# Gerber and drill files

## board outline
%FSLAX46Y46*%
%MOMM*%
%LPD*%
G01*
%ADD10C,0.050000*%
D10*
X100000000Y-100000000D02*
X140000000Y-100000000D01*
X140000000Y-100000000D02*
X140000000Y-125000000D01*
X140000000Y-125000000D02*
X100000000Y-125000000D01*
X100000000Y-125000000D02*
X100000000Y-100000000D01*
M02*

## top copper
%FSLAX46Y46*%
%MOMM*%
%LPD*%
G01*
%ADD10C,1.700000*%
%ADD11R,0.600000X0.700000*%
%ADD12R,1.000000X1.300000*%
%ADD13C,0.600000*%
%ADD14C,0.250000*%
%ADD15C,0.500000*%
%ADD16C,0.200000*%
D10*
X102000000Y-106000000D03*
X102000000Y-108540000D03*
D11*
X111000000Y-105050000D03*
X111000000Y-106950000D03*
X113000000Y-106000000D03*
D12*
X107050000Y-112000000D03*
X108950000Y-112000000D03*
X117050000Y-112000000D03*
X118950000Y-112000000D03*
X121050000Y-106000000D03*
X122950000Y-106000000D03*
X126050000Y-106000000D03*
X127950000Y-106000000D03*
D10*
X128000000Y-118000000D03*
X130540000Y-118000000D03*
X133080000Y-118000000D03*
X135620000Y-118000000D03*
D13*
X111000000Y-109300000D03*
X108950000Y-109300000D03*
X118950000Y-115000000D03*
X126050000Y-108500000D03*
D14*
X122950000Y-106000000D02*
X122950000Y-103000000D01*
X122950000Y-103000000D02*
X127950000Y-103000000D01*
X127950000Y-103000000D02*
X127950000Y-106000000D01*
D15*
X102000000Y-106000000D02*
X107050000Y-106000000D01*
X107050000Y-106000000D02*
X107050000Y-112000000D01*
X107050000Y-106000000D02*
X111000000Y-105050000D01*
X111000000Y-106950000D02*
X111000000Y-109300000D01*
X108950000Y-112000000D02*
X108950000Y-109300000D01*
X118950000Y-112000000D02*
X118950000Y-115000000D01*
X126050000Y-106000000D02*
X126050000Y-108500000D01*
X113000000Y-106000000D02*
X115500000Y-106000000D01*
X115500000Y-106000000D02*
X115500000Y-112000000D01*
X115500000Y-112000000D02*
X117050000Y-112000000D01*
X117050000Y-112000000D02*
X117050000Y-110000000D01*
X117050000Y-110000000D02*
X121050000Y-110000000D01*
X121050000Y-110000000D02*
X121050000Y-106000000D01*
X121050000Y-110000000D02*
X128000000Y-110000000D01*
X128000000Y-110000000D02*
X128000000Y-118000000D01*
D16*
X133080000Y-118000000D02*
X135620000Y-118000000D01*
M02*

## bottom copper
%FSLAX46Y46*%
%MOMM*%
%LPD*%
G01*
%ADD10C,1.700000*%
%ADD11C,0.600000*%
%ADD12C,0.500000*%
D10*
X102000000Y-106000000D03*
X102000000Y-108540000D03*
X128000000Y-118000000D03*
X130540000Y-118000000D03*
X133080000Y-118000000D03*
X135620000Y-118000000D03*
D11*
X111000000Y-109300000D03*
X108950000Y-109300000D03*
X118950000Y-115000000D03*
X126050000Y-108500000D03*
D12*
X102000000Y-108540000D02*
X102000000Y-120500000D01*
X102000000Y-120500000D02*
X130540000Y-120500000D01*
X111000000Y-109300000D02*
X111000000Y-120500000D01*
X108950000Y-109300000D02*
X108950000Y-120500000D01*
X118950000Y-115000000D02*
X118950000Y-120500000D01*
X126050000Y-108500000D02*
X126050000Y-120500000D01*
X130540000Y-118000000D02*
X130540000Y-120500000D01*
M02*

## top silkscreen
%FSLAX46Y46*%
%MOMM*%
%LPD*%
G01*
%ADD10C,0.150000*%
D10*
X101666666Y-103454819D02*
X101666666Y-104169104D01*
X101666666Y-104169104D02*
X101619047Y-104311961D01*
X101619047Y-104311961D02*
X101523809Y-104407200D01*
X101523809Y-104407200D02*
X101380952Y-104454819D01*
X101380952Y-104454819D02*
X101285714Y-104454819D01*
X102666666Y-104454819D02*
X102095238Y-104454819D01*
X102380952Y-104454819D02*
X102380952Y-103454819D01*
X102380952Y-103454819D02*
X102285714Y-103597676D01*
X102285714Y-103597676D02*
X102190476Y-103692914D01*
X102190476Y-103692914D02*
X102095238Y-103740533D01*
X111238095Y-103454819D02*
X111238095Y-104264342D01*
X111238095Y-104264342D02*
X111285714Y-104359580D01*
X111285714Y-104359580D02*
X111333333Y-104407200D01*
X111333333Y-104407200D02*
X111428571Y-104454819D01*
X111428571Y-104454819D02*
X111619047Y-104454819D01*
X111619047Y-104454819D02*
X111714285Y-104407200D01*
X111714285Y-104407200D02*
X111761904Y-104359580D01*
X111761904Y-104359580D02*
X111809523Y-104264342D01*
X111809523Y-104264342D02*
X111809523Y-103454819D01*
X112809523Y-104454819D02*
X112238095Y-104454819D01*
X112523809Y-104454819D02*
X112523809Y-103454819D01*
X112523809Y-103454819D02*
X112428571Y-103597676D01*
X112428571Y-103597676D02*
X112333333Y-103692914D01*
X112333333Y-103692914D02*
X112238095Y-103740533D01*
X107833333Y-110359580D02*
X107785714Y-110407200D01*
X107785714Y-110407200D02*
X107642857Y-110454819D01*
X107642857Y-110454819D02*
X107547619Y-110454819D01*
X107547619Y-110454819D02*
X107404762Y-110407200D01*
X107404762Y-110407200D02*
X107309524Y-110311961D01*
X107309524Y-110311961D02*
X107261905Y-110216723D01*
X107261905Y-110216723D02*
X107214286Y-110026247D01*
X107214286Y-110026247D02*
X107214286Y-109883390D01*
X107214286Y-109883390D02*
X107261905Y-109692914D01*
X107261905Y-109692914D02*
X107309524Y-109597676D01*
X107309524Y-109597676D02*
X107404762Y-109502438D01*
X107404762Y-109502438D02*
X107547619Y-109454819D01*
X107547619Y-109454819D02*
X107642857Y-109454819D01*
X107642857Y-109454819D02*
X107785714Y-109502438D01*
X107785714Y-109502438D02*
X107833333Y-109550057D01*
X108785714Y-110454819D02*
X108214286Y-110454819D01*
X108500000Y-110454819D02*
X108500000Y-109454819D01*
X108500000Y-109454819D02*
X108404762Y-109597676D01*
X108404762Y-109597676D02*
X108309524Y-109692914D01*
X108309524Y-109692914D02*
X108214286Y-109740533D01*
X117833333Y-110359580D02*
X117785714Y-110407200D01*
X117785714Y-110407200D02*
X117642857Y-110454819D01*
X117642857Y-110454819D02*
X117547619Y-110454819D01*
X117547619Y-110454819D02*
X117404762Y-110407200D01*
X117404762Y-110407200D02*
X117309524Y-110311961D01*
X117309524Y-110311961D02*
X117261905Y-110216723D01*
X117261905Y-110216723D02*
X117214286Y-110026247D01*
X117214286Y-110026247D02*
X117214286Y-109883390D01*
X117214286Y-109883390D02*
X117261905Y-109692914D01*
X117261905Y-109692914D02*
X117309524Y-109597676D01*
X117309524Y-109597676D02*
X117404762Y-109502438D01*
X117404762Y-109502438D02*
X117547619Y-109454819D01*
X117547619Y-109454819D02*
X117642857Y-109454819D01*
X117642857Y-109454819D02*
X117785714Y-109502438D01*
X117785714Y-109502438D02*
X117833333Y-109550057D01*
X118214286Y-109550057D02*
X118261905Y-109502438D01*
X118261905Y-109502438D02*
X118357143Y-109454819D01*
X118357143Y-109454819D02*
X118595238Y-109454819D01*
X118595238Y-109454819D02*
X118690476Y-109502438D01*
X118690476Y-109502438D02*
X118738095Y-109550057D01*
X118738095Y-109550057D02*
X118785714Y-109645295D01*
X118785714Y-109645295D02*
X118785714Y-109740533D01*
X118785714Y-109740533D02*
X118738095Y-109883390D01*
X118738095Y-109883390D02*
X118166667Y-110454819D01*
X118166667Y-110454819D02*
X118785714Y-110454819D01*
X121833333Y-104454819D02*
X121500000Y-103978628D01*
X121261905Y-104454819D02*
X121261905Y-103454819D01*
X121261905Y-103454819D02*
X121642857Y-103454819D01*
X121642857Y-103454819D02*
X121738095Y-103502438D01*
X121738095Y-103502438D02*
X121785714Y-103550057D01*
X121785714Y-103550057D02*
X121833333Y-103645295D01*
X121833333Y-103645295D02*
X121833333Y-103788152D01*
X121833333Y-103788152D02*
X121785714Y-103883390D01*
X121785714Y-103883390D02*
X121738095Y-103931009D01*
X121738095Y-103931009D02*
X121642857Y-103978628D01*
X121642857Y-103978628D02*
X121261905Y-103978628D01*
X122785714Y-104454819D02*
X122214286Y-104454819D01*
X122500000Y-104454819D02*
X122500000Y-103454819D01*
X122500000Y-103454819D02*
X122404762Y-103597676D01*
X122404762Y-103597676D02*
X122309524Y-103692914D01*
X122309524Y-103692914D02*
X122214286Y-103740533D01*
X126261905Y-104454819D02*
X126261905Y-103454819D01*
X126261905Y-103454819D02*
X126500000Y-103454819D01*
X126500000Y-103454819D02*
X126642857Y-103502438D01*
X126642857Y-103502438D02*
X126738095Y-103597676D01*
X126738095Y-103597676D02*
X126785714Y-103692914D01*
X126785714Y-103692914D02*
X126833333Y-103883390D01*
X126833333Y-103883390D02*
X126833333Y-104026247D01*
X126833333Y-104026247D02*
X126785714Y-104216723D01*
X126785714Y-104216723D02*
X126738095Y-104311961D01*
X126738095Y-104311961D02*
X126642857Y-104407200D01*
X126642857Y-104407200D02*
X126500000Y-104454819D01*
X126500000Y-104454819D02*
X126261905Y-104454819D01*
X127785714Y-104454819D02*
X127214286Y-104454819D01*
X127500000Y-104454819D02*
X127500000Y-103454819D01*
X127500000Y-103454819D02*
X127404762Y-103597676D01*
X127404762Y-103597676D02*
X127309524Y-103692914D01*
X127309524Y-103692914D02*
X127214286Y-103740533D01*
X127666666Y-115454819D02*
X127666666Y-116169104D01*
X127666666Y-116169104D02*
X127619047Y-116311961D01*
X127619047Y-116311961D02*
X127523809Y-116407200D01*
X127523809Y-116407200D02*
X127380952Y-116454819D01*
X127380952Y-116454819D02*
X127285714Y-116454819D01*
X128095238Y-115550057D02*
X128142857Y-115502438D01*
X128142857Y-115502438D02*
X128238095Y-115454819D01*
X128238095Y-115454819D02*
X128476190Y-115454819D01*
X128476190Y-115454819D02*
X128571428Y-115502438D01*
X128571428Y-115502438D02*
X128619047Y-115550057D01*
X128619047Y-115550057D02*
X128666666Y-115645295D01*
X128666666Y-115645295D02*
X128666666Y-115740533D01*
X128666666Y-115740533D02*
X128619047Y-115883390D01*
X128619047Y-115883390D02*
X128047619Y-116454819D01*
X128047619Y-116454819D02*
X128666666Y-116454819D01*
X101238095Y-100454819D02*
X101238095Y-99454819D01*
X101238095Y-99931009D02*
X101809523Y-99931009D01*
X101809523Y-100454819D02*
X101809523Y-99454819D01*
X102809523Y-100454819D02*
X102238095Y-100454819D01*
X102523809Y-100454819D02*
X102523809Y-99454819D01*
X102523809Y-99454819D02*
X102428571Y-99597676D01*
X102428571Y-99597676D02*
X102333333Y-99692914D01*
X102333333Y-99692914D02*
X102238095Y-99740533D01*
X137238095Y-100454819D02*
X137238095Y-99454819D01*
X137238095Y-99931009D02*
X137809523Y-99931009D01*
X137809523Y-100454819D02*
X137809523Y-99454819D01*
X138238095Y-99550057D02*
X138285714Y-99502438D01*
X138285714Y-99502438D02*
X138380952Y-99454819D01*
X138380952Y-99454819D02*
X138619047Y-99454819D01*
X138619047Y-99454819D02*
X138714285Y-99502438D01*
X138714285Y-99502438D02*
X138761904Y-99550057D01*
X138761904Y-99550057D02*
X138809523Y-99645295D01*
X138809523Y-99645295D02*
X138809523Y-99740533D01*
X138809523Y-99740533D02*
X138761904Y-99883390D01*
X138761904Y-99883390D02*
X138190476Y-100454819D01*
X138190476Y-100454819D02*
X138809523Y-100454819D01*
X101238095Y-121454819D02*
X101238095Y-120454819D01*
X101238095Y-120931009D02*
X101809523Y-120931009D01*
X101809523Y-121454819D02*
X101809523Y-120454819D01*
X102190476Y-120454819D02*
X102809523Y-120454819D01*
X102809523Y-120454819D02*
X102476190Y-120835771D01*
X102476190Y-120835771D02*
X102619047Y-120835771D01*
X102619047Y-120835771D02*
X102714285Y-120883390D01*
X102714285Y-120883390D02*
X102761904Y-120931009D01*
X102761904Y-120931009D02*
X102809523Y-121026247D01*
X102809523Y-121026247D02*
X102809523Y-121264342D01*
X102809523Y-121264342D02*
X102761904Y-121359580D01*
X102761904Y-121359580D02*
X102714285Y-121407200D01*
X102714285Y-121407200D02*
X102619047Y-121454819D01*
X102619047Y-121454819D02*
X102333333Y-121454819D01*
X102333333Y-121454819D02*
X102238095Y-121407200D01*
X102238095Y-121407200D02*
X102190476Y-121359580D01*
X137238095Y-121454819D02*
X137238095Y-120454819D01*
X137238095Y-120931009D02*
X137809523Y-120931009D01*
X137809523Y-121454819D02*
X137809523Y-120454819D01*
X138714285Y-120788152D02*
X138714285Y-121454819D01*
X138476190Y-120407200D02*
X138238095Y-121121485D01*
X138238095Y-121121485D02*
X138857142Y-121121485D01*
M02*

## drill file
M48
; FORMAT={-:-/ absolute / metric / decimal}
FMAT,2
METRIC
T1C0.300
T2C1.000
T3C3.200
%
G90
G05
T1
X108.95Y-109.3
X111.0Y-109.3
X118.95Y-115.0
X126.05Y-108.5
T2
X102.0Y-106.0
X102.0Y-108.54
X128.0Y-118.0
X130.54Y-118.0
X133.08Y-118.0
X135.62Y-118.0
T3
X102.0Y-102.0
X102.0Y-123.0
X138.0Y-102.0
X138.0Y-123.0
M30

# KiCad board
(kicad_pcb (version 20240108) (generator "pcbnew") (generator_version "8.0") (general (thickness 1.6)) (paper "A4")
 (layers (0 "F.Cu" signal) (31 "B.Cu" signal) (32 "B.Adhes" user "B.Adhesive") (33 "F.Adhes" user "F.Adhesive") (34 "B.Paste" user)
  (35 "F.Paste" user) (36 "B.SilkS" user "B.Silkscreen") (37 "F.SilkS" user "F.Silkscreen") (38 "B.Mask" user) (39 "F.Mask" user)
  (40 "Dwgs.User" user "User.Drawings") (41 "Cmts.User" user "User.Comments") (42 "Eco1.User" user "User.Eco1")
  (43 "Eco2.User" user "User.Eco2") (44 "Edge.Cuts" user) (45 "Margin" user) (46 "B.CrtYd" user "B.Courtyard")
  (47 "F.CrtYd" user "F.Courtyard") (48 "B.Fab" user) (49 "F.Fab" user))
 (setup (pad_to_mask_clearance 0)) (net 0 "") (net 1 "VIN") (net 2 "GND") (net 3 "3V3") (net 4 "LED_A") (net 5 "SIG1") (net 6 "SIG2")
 (gr_line (start 100 100) (end 140 100) (stroke (width 0.05) (type default)) (layer "Edge.Cuts"))
 (gr_line (start 140 100) (end 140 125) (stroke (width 0.05) (type default)) (layer "Edge.Cuts"))
 (gr_line (start 140 125) (end 100 125) (stroke (width 0.05) (type default)) (layer "Edge.Cuts"))
 (gr_line (start 100 125) (end 100 100) (stroke (width 0.05) (type default)) (layer "Edge.Cuts"))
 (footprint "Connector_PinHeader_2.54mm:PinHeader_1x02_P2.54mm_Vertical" (layer "F.Cu") (at 102 106)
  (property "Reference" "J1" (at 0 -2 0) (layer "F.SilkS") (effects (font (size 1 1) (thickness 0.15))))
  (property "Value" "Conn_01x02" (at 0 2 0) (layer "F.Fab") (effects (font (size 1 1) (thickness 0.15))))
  (pad "1" thru_hole circle (at 0 0) (size 1.7 1.7) (drill 1) (layers "*.Cu" "*.Mask") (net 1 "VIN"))
  (pad "2" thru_hole circle (at 0 2.54) (size 1.7 1.7) (drill 1) (layers "*.Cu" "*.Mask") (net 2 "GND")))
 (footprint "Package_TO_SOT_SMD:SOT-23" (layer "F.Cu") (at 112 106)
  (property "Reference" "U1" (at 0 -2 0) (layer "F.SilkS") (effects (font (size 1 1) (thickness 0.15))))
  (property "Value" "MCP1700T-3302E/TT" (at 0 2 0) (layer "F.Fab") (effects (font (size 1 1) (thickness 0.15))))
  (pad "1" smd rect (at -1 -0.95) (size 0.6 0.7) (layers "F.Cu" "F.Paste" "F.Mask") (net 1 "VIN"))
  (pad "2" smd rect (at -1 0.95) (size 0.6 0.7) (layers "F.Cu" "F.Paste" "F.Mask") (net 2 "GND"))
  (pad "3" smd rect (at 1 0) (size 0.6 0.7) (layers "F.Cu" "F.Paste" "F.Mask") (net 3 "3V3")))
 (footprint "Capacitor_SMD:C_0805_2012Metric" (layer "F.Cu") (at 108 112)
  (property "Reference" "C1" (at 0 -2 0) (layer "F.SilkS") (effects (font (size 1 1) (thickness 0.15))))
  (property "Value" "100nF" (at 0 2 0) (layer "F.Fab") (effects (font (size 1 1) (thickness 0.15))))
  (pad "1" smd rect (at -0.95 0) (size 1 1.3) (layers "F.Cu" "F.Paste" "F.Mask") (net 1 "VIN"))
  (pad "2" smd rect (at 0.95 0) (size 1 1.3) (layers "F.Cu" "F.Paste" "F.Mask") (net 2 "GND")))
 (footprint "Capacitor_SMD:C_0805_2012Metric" (layer "F.Cu") (at 118 112)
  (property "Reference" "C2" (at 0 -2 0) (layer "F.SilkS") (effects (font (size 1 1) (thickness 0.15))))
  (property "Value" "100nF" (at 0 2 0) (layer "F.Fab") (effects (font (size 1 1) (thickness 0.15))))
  (pad "1" smd rect (at -0.95 0) (size 1 1.3) (layers "F.Cu" "F.Paste" "F.Mask") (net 3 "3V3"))
  (pad "2" smd rect (at 0.95 0) (size 1 1.3) (layers "F.Cu" "F.Paste" "F.Mask") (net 2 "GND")))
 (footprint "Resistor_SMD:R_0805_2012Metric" (layer "F.Cu") (at 122 106)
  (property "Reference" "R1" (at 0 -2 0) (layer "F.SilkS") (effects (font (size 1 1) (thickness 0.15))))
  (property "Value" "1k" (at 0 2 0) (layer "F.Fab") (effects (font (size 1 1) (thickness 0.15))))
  (pad "1" smd rect (at -0.95 0) (size 1 1.3) (layers "F.Cu" "F.Paste" "F.Mask") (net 3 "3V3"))
  (pad "2" smd rect (at 0.95 0) (size 1 1.3) (layers "F.Cu" "F.Paste" "F.Mask") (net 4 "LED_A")))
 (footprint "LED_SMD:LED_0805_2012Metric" (layer "F.Cu") (at 127 106)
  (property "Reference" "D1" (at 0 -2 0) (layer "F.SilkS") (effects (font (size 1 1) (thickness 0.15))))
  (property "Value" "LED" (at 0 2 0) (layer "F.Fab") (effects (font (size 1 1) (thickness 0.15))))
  (pad "1" smd rect (at -0.95 0) (size 1 1.3) (layers "F.Cu" "F.Paste" "F.Mask") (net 2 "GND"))
  (pad "2" smd rect (at 0.95 0) (size 1 1.3) (layers "F.Cu" "F.Paste" "F.Mask") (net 4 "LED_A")))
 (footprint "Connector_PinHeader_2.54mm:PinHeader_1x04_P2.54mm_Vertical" (layer "F.Cu") (at 128 118)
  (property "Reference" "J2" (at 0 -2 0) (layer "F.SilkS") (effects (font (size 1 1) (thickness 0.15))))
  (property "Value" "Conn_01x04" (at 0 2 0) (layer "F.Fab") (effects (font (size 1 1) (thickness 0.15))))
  (pad "1" thru_hole circle (at 0 0) (size 1.7 1.7) (drill 1) (layers "*.Cu" "*.Mask") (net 3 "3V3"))
  (pad "2" thru_hole circle (at 2.54 0) (size 1.7 1.7) (drill 1) (layers "*.Cu" "*.Mask") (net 2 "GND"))
  (pad "3" thru_hole circle (at 5.08 0) (size 1.7 1.7) (drill 1) (layers "*.Cu" "*.Mask") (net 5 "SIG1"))
  (pad "4" thru_hole circle (at 7.62 0) (size 1.7 1.7) (drill 1) (layers "*.Cu" "*.Mask") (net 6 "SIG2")))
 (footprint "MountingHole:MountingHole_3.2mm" (layer "F.Cu") (at 102 102)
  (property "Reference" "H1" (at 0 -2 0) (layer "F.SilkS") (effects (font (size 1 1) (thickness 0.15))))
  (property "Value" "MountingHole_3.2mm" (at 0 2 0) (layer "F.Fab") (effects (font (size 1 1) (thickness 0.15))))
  (pad "1" np_thru_hole circle (at 0 0) (size 3.2 3.2) (drill 3.2) (layers "*.Cu" "*.Mask")))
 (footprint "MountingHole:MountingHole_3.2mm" (layer "F.Cu") (at 138 102)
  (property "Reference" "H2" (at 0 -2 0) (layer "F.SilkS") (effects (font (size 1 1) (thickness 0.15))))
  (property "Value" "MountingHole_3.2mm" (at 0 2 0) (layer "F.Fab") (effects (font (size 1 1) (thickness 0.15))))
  (pad "1" np_thru_hole circle (at 0 0) (size 3.2 3.2) (drill 3.2) (layers "*.Cu" "*.Mask")))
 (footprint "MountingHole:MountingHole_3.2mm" (layer "F.Cu") (at 102 123)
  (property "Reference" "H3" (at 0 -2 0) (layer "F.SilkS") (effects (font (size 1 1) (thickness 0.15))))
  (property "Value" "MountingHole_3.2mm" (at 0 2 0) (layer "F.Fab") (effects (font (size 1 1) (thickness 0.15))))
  (pad "1" np_thru_hole circle (at 0 0) (size 3.2 3.2) (drill 3.2) (layers "*.Cu" "*.Mask")))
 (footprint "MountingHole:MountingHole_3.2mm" (layer "F.Cu") (at 138 123)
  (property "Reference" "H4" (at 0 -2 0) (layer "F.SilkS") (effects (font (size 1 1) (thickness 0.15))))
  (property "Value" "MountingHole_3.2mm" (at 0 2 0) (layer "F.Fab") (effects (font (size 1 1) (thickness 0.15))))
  (pad "1" np_thru_hole circle (at 0 0) (size 3.2 3.2) (drill 3.2) (layers "*.Cu" "*.Mask")))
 (segment (start 122.95 106) (end 122.95 103) (width 0.25) (layer "F.Cu") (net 4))
 (segment (start 122.95 103) (end 127.95 103) (width 0.25) (layer "F.Cu") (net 4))
 (segment (start 127.95 103) (end 127.95 106) (width 0.25) (layer "F.Cu") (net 4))
 (segment (start 102 106) (end 107.05 106) (width 0.5) (layer "F.Cu") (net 1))
 (segment (start 107.05 106) (end 107.05 112) (width 0.5) (layer "F.Cu") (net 1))
 (segment (start 107.05 106) (end 111 105.05) (width 0.5) (layer "F.Cu") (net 1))
 (segment (start 111 106.95) (end 111 109.3) (width 0.5) (layer "F.Cu") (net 2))
 (segment (start 108.95 112) (end 108.95 109.3) (width 0.5) (layer "F.Cu") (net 2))
 (segment (start 118.95 112) (end 118.95 115) (width 0.5) (layer "F.Cu") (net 2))
 (segment (start 126.05 106) (end 126.05 108.5) (width 0.5) (layer "F.Cu") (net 2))
 (segment (start 113 106) (end 115.5 106) (width 0.5) (layer "F.Cu") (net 3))
 (segment (start 115.5 106) (end 115.5 112) (width 0.5) (layer "F.Cu") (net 3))
 (segment (start 115.5 112) (end 117.05 112) (width 0.5) (layer "F.Cu") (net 3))
 (segment (start 117.05 112) (end 117.05 110) (width 0.5) (layer "F.Cu") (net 3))
 (segment (start 117.05 110) (end 121.05 110) (width 0.5) (layer "F.Cu") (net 3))
 (segment (start 121.05 110) (end 121.05 106) (width 0.5) (layer "F.Cu") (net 3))
 (segment (start 121.05 110) (end 128 110) (width 0.5) (layer "F.Cu") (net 3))
 (segment (start 128 110) (end 128 118) (width 0.5) (layer "F.Cu") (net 3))
 (segment (start 102 108.54) (end 102 120.5) (width 0.5) (layer "B.Cu") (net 2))
 (segment (start 102 120.5) (end 130.54 120.5) (width 0.5) (layer "B.Cu") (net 2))
 (segment (start 111 109.3) (end 111 120.5) (width 0.5) (layer "B.Cu") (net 2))
 (segment (start 108.95 109.3) (end 108.95 120.5) (width 0.5) (layer "B.Cu") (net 2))
 (segment (start 118.95 115) (end 118.95 120.5) (width 0.5) (layer "B.Cu") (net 2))
 (segment (start 126.05 108.5) (end 126.05 120.5) (width 0.5) (layer "B.Cu") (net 2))
 (segment (start 130.54 118) (end 130.54 120.5) (width 0.5) (layer "B.Cu") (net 2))
 (via (at 111 109.3) (size 0.6) (drill 0.3) (layers "F.Cu" "B.Cu") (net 2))
 (via (at 108.95 109.3) (size 0.6) (drill 0.3) (layers "F.Cu" "B.Cu") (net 2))
 (via (at 118.95 115) (size 0.6) (drill 0.3) (layers "F.Cu" "B.Cu") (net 2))
 (via (at 126.05 108.5) (size 0.6) (drill 0.3) (layers "F.Cu" "B.Cu") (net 2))
 (segment (start 133.08 118) (end 135.62 118) (width 0.2) (layer "F.Cu") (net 5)))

